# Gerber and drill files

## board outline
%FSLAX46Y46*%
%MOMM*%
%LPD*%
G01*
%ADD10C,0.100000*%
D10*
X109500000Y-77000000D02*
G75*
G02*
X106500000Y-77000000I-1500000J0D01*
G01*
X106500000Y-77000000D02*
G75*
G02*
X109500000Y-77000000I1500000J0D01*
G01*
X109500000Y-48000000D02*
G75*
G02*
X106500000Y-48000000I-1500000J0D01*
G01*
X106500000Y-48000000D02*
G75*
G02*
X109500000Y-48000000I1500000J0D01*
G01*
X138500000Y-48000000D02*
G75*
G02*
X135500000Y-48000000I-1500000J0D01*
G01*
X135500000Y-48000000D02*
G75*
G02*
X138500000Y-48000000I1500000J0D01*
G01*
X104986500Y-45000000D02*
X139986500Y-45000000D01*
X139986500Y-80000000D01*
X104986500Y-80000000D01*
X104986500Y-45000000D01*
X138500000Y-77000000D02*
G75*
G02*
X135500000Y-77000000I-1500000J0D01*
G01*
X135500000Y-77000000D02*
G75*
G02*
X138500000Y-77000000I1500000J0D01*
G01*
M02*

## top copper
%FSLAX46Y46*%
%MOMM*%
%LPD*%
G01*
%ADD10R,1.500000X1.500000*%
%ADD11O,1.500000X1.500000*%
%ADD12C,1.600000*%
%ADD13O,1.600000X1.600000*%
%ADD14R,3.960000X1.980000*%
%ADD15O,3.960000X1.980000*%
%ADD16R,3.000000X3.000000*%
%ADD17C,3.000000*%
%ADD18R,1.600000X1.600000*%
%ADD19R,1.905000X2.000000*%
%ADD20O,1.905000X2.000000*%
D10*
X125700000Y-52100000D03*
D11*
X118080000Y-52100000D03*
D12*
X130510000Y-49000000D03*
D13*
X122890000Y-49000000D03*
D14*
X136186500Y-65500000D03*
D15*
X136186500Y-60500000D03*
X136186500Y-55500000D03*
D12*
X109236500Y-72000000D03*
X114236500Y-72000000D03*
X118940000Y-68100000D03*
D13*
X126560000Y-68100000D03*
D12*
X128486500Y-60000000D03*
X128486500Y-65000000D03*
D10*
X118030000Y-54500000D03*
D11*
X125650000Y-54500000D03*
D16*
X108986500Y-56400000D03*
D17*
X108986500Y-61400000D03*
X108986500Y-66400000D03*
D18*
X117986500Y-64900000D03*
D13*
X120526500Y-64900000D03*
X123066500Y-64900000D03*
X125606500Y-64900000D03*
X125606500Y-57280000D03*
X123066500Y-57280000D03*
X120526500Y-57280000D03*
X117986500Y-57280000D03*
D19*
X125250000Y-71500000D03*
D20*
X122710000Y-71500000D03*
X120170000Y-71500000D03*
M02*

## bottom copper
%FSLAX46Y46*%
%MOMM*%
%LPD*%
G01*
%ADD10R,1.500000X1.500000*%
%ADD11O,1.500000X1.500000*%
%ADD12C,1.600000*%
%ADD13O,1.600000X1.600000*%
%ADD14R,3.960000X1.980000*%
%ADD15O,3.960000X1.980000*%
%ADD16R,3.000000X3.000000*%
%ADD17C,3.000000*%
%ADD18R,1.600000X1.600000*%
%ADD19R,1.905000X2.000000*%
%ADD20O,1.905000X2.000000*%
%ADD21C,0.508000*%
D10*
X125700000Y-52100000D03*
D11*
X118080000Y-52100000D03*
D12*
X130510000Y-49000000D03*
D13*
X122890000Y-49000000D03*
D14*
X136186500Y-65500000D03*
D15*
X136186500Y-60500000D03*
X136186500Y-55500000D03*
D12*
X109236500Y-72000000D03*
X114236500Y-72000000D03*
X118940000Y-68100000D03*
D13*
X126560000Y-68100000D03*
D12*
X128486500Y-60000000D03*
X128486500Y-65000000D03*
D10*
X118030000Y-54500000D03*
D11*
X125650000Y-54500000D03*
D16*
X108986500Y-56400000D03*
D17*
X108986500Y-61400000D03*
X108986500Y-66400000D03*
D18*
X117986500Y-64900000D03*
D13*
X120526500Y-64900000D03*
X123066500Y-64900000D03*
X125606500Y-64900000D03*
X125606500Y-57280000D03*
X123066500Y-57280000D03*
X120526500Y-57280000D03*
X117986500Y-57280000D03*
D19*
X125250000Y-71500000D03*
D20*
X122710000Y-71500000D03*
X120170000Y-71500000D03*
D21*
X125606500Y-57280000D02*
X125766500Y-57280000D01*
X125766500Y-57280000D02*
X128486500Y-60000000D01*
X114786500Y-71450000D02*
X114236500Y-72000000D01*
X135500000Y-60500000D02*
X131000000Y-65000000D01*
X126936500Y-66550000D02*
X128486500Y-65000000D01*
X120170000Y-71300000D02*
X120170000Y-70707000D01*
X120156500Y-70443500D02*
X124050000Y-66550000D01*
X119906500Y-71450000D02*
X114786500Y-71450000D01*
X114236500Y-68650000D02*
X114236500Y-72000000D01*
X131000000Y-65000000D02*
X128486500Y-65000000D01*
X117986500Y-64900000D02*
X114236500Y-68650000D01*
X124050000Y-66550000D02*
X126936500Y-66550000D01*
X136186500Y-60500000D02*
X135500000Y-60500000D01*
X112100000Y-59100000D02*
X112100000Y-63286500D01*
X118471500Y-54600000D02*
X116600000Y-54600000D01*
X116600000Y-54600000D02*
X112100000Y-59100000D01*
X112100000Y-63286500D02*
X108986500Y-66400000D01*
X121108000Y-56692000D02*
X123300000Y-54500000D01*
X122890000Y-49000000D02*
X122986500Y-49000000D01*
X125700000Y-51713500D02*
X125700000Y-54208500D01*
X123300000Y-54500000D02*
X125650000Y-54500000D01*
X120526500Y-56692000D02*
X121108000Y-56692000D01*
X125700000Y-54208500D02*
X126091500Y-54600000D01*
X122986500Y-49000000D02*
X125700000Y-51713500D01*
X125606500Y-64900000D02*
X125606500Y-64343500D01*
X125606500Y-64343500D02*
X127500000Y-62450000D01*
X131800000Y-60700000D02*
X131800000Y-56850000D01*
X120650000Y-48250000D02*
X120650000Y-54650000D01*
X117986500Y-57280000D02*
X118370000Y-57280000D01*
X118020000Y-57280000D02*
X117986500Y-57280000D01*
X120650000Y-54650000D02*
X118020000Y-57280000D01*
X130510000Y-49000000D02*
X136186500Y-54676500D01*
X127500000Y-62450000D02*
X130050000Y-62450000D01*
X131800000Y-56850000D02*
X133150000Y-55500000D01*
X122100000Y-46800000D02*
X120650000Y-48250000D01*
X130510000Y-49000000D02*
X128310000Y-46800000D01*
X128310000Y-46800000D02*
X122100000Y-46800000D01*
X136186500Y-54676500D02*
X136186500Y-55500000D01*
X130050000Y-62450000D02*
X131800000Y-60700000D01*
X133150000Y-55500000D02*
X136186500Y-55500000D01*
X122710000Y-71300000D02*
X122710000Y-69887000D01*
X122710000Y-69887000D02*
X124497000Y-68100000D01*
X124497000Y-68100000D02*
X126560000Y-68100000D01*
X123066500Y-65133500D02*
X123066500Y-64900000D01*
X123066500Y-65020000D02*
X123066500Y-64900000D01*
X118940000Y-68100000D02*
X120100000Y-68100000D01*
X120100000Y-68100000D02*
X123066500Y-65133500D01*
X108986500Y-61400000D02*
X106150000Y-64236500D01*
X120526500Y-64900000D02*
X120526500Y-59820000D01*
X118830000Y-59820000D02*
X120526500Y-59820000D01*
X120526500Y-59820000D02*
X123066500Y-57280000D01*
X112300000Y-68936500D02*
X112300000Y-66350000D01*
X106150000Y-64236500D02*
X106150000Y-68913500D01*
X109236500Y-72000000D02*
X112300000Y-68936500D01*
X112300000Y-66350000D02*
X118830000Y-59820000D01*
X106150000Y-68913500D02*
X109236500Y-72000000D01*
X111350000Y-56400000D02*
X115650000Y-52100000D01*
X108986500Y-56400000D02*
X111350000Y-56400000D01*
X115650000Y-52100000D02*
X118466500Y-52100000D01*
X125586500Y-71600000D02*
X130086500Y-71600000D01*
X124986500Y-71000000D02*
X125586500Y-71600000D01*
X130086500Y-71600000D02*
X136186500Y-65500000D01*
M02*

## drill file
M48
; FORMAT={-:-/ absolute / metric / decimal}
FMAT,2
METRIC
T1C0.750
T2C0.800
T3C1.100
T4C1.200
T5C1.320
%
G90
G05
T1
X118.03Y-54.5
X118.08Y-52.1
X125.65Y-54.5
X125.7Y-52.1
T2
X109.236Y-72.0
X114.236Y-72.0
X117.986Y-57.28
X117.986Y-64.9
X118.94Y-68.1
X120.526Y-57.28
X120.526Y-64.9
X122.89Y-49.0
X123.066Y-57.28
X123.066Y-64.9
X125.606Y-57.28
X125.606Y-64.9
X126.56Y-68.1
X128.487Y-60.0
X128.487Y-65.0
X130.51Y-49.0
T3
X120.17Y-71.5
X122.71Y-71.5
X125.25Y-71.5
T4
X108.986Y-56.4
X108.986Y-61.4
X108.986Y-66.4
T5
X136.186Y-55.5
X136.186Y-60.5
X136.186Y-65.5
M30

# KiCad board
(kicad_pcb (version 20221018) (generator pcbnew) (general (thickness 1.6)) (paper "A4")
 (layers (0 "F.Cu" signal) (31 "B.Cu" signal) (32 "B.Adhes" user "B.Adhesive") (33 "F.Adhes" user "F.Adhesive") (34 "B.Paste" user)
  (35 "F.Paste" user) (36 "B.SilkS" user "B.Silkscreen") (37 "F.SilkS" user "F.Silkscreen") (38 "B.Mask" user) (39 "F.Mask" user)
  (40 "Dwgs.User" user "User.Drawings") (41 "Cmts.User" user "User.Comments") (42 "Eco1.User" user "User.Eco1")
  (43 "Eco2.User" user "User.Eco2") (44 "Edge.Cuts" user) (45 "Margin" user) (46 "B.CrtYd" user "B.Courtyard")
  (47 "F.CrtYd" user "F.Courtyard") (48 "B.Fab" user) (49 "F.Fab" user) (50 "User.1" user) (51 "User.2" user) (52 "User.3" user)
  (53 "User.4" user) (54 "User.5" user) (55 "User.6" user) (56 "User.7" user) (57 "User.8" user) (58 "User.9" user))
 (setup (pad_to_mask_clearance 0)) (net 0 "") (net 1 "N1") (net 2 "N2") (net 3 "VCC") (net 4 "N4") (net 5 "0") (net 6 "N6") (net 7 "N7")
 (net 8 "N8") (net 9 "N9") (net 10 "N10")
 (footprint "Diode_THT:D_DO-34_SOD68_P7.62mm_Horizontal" (layer "F.Cu") (at 125.7 52.1 180)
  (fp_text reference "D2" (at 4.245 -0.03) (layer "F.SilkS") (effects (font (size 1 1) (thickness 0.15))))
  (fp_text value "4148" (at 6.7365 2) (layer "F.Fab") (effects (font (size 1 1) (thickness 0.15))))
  (pad "1" thru_hole rect (at 0 0 180) (size 1.5 1.5) (drill 0.75) (layers "*.Cu" "*.Mask") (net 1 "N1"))
  (pad "2" thru_hole oval (at 7.62 0 180) (size 1.5 1.5) (drill 0.75) (layers "*.Cu" "*.Mask") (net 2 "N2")))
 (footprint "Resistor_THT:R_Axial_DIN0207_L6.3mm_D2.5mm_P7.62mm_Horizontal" (layer "F.Cu") (at 130.51 49 180)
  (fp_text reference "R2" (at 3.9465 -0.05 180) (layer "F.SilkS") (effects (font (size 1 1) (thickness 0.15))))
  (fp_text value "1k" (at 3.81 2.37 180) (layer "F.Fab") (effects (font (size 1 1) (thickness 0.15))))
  (pad "1" thru_hole circle (at 0 0 180) (size 1.6 1.6) (drill 0.8) (layers "*.Cu" "*.Mask") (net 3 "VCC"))
  (pad "2" thru_hole oval (at 7.62 0 180) (size 1.6 1.6) (drill 0.8) (layers "*.Cu" "*.Mask") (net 1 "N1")))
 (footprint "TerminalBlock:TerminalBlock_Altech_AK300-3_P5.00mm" (layer "F.Cu") (at 136.1865 65.5 90)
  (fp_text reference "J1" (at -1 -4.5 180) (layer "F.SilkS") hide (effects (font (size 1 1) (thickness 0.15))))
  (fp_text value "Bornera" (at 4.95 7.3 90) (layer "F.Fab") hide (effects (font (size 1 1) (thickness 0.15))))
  (pad "1" thru_hole rect (at 0 0 90) (size 1.98 3.96) (drill 1.32) (layers "*.Cu" "*.Mask") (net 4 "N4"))
  (pad "2" thru_hole oval (at 5 0 90) (size 1.98 3.96) (drill 1.32) (layers "*.Cu" "*.Mask") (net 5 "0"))
  (pad "3" thru_hole oval (at 10 0 90) (size 1.98 3.96) (drill 1.32) (layers "*.Cu" "*.Mask") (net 3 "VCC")))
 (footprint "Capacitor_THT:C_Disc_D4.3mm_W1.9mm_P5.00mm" (layer "F.Cu") (at 109.2365 72)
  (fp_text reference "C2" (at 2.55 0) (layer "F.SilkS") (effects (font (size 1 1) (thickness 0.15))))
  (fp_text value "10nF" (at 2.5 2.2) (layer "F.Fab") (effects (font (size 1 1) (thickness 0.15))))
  (pad "1" thru_hole circle (at 0 0) (size 1.6 1.6) (drill 0.8) (layers "*.Cu" "*.Mask") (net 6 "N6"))
  (pad "2" thru_hole circle (at 5 0) (size 1.6 1.6) (drill 0.8) (layers "*.Cu" "*.Mask") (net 5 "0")))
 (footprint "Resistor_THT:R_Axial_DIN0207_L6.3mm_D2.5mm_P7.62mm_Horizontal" (layer "F.Cu") (at 118.94 68.1)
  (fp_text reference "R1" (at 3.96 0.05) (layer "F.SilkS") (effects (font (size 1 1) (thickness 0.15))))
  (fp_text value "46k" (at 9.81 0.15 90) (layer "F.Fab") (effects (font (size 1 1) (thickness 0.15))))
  (pad "1" thru_hole circle (at 0 0) (size 1.6 1.6) (drill 0.8) (layers "*.Cu" "*.Mask") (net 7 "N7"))
  (pad "2" thru_hole oval (at 7.62 0) (size 1.6 1.6) (drill 0.8) (layers "*.Cu" "*.Mask") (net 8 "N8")))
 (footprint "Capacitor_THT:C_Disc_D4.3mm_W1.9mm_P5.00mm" (layer "F.Cu") (at 128.4865 60 -90)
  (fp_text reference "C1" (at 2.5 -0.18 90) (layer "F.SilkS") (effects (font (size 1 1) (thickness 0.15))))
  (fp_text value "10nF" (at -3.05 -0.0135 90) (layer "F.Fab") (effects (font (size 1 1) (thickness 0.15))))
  (pad "1" thru_hole circle (at 0 0 270) (size 1.6 1.6) (drill 0.8) (layers "*.Cu" "*.Mask") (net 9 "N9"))
  (pad "2" thru_hole circle (at 5 0 270) (size 1.6 1.6) (drill 0.8) (layers "*.Cu" "*.Mask") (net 5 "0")))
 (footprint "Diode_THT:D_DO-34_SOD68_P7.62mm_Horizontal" (layer "F.Cu") (at 118.03 54.5)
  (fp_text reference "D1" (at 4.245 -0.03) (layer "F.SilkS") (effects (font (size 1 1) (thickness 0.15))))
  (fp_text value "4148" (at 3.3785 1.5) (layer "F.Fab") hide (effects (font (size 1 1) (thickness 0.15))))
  (pad "1" thru_hole rect (at 0 0) (size 1.5 1.5) (drill 0.75) (layers "*.Cu" "*.Mask") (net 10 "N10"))
  (pad "2" thru_hole oval (at 7.62 0) (size 1.5 1.5) (drill 0.75) (layers "*.Cu" "*.Mask") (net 1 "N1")))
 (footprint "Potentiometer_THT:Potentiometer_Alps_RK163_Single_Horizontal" (layer "F.Cu") (at 108.9865 56.4)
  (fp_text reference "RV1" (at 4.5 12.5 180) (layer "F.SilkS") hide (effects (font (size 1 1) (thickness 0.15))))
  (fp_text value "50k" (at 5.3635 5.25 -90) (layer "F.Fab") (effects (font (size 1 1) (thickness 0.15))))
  (pad "1" thru_hole rect (at 0 0 180) (size 3 3) (drill 1.2) (layers "*.Cu" "*.Mask") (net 2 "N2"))
  (pad "2" thru_hole circle (at 0 5 180) (size 3 3) (drill 1.2) (layers "*.Cu" "*.Mask") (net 6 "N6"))
  (pad "3" thru_hole circle (at 0 10 180) (size 3 3) (drill 1.2) (layers "*.Cu" "*.Mask") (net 10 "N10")))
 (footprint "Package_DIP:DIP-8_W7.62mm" (layer "F.Cu") (at 117.9865 64.9 90)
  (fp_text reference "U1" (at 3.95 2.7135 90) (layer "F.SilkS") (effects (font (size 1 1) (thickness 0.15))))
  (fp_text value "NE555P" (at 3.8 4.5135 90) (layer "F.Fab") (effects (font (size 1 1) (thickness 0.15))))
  (pad "1" thru_hole rect (at 0 0 90) (size 1.6 1.6) (drill 0.8) (layers "*.Cu" "*.Mask") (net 5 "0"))
  (pad "2" thru_hole oval (at 0 2.54 90) (size 1.6 1.6) (drill 0.8) (layers "*.Cu" "*.Mask") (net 6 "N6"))
  (pad "3" thru_hole oval (at 0 5.08 90) (size 1.6 1.6) (drill 0.8) (layers "*.Cu" "*.Mask") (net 7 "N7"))
  (pad "4" thru_hole oval (at 0 7.62 90) (size 1.6 1.6) (drill 0.8) (layers "*.Cu" "*.Mask") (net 3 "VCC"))
  (pad "5" thru_hole oval (at 7.62 7.62 90) (size 1.6 1.6) (drill 0.8) (layers "*.Cu" "*.Mask") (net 9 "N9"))
  (pad "6" thru_hole oval (at 7.62 5.08 90) (size 1.6 1.6) (drill 0.8) (layers "*.Cu" "*.Mask") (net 6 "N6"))
  (pad "7" thru_hole oval (at 7.62 2.54 90) (size 1.6 1.6) (drill 0.8) (layers "*.Cu" "*.Mask") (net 1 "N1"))
  (pad "8" thru_hole oval (at 7.62 0 90) (size 1.6 1.6) (drill 0.8) (layers "*.Cu" "*.Mask") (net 3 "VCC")))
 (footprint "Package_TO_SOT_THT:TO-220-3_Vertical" (layer "F.Cu") (at 125.25 71.5 180)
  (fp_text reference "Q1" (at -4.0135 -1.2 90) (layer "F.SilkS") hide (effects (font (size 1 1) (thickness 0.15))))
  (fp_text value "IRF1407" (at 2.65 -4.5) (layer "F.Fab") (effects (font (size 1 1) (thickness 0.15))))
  (pad "1" thru_hole rect (at 0 0 180) (size 1.905 2) (drill 1.1) (layers "*.Cu" "*.Mask") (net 4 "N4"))
  (pad "2" thru_hole oval (at 2.54 0 180) (size 1.905 2) (drill 1.1) (layers "*.Cu" "*.Mask") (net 8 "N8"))
  (pad "3" thru_hole oval (at 5.08 0 180) (size 1.905 2) (drill 1.1) (layers "*.Cu" "*.Mask") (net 5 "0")))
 (gr_circle (center 108 77) (end 109.5 77) (stroke (width 0.1) (type default)) (fill none) (layer "Edge.Cuts"))
 (gr_circle (center 108 48) (end 109.5 48) (stroke (width 0.1) (type default)) (fill none) (layer "Edge.Cuts"))
 (gr_circle (center 137 48) (end 138.5 48) (stroke (width 0.1) (type default)) (fill none) (layer "Edge.Cuts"))
 (gr_rect (start 104.9865 45) (end 139.9865 80) (stroke (width 0.1) (type default)) (fill none) (layer "Edge.Cuts"))
 (gr_circle (center 137 77) (end 138.5 77) (stroke (width 0.1) (type default)) (fill none) (layer "Edge.Cuts"))
 (segment (start 125.6065 57.28) (end 125.7665 57.28) (width 0.508) (layer "B.Cu") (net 9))
 (segment (start 125.7665 57.28) (end 128.4865 60) (width 0.508) (layer "B.Cu") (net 9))
 (segment (start 114.7865 71.45) (end 114.2365 72) (width 0.508) (layer "B.Cu") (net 5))
 (segment (start 135.5 60.5) (end 131 65) (width 0.508) (layer "B.Cu") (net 5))
 (segment (start 126.9365 66.55) (end 128.4865 65) (width 0.508) (layer "B.Cu") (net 5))
 (segment (start 120.17 71.3) (end 120.17 70.707) (width 0.508) (layer "B.Cu") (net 5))
 (segment (start 120.1565 70.4435) (end 124.05 66.55) (width 0.508) (layer "B.Cu") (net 5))
 (segment (start 119.9065 71.45) (end 114.7865 71.45) (width 0.508) (layer "B.Cu") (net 5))
 (segment (start 114.2365 68.65) (end 114.2365 72) (width 0.508) (layer "B.Cu") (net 5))
 (segment (start 131 65) (end 128.4865 65) (width 0.508) (layer "B.Cu") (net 5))
 (segment (start 117.9865 64.9) (end 114.2365 68.65) (width 0.508) (layer "B.Cu") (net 5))
 (segment (start 124.05 66.55) (end 126.9365 66.55) (width 0.508) (layer "B.Cu") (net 5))
 (segment (start 136.1865 60.5) (end 135.5 60.5) (width 0.508) (layer "B.Cu") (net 5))
 (segment (start 112.1 59.1) (end 112.1 63.2865) (width 0.508) (layer "B.Cu") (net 10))
 (segment (start 118.4715 54.6) (end 116.6 54.6) (width 0.508) (layer "B.Cu") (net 10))
 (segment (start 116.6 54.6) (end 112.1 59.1) (width 0.508) (layer "B.Cu") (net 10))
 (segment (start 112.1 63.2865) (end 108.9865 66.4) (width 0.508) (layer "B.Cu") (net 10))
 (segment (start 121.108 56.692) (end 123.3 54.5) (width 0.508) (layer "B.Cu") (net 1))
 (segment (start 122.89 49) (end 122.9865 49) (width 0.508) (layer "B.Cu") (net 1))
 (segment (start 125.7 51.7135) (end 125.7 54.2085) (width 0.508) (layer "B.Cu") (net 1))
 (segment (start 123.3 54.5) (end 125.65 54.5) (width 0.508) (layer "B.Cu") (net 1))
 (segment (start 120.5265 56.692) (end 121.108 56.692) (width 0.508) (layer "B.Cu") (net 1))
 (segment (start 125.7 54.2085) (end 126.0915 54.6) (width 0.508) (layer "B.Cu") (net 1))
 (segment (start 122.9865 49) (end 125.7 51.7135) (width 0.508) (layer "B.Cu") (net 1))
 (segment (start 125.6065 64.9) (end 125.6065 64.3435) (width 0.508) (layer "B.Cu") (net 3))
 (segment (start 125.6065 64.3435) (end 127.5 62.45) (width 0.508) (layer "B.Cu") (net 3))
 (segment (start 131.8 60.7) (end 131.8 56.85) (width 0.508) (layer "B.Cu") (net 3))
 (segment (start 120.65 48.25) (end 120.65 54.65) (width 0.508) (layer "B.Cu") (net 3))
 (segment (start 117.9865 57.28) (end 118.37 57.28) (width 0.508) (layer "B.Cu") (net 3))
 (segment (start 118.02 57.28) (end 117.9865 57.28) (width 0.508) (layer "B.Cu") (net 3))
 (segment (start 120.65 54.65) (end 118.02 57.28) (width 0.508) (layer "B.Cu") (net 3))
 (segment (start 130.51 49) (end 136.1865 54.6765) (width 0.508) (layer "B.Cu") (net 3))
 (segment (start 127.5 62.45) (end 130.05 62.45) (width 0.508) (layer "B.Cu") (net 3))
 (segment (start 131.8 56.85) (end 133.15 55.5) (width 0.508) (layer "B.Cu") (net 3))
 (segment (start 122.1 46.8) (end 120.65 48.25) (width 0.508) (layer "B.Cu") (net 3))
 (segment (start 130.51 49) (end 128.31 46.8) (width 0.508) (layer "B.Cu") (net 3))
 (segment (start 128.31 46.8) (end 122.1 46.8) (width 0.508) (layer "B.Cu") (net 3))
 (segment (start 136.1865 54.6765) (end 136.1865 55.5) (width 0.508) (layer "B.Cu") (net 3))
 (segment (start 130.05 62.45) (end 131.8 60.7) (width 0.508) (layer "B.Cu") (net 3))
 (segment (start 133.15 55.5) (end 136.1865 55.5) (width 0.508) (layer "B.Cu") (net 3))
 (segment (start 122.71 71.3) (end 122.71 69.887) (width 0.508) (layer "B.Cu") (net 8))
 (segment (start 122.71 69.887) (end 124.497 68.1) (width 0.508) (layer "B.Cu") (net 8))
 (segment (start 124.497 68.1) (end 126.56 68.1) (width 0.508) (layer "B.Cu") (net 8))
 (segment (start 123.0665 65.1335) (end 123.0665 64.9) (width 0.508) (layer "B.Cu") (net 7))
 (segment (start 123.0665 65.02) (end 123.0665 64.9) (width 0.508) (layer "B.Cu") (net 7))
 (segment (start 118.94 68.1) (end 120.1 68.1) (width 0.508) (layer "B.Cu") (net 7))
 (segment (start 120.1 68.1) (end 123.0665 65.1335) (width 0.508) (layer "B.Cu") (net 7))
 (segment (start 108.9865 61.4) (end 106.15 64.2365) (width 0.508) (layer "B.Cu") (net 6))
 (segment (start 120.5265 64.9) (end 120.5265 59.82) (width 0.508) (layer "B.Cu") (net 6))
 (segment (start 118.83 59.82) (end 120.5265 59.82) (width 0.508) (layer "B.Cu") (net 6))
 (segment (start 120.5265 59.82) (end 123.0665 57.28) (width 0.508) (layer "B.Cu") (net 6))
 (segment (start 112.3 68.9365) (end 112.3 66.35) (width 0.508) (layer "B.Cu") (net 6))
 (segment (start 106.15 64.2365) (end 106.15 68.9135) (width 0.508) (layer "B.Cu") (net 6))
 (segment (start 109.2365 72) (end 112.3 68.9365) (width 0.508) (layer "B.Cu") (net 6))
 (segment (start 112.3 66.35) (end 118.83 59.82) (width 0.508) (layer "B.Cu") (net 6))
 (segment (start 106.15 68.9135) (end 109.2365 72) (width 0.508) (layer "B.Cu") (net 6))
 (segment (start 111.35 56.4) (end 115.65 52.1) (width 0.508) (layer "B.Cu") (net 2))
 (segment (start 108.9865 56.4) (end 111.35 56.4) (width 0.508) (layer "B.Cu") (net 2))
 (segment (start 115.65 52.1) (end 118.4665 52.1) (width 0.508) (layer "B.Cu") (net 2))
 (segment (start 125.5865 71.6) (end 130.0865 71.6) (width 0.508) (layer "B.Cu") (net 4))
 (segment (start 124.9865 71) (end 125.5865 71.6) (width 0.508) (layer "B.Cu") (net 4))
 (segment (start 130.0865 71.6) (end 136.1865 65.5) (width 0.508) (layer "B.Cu") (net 4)))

